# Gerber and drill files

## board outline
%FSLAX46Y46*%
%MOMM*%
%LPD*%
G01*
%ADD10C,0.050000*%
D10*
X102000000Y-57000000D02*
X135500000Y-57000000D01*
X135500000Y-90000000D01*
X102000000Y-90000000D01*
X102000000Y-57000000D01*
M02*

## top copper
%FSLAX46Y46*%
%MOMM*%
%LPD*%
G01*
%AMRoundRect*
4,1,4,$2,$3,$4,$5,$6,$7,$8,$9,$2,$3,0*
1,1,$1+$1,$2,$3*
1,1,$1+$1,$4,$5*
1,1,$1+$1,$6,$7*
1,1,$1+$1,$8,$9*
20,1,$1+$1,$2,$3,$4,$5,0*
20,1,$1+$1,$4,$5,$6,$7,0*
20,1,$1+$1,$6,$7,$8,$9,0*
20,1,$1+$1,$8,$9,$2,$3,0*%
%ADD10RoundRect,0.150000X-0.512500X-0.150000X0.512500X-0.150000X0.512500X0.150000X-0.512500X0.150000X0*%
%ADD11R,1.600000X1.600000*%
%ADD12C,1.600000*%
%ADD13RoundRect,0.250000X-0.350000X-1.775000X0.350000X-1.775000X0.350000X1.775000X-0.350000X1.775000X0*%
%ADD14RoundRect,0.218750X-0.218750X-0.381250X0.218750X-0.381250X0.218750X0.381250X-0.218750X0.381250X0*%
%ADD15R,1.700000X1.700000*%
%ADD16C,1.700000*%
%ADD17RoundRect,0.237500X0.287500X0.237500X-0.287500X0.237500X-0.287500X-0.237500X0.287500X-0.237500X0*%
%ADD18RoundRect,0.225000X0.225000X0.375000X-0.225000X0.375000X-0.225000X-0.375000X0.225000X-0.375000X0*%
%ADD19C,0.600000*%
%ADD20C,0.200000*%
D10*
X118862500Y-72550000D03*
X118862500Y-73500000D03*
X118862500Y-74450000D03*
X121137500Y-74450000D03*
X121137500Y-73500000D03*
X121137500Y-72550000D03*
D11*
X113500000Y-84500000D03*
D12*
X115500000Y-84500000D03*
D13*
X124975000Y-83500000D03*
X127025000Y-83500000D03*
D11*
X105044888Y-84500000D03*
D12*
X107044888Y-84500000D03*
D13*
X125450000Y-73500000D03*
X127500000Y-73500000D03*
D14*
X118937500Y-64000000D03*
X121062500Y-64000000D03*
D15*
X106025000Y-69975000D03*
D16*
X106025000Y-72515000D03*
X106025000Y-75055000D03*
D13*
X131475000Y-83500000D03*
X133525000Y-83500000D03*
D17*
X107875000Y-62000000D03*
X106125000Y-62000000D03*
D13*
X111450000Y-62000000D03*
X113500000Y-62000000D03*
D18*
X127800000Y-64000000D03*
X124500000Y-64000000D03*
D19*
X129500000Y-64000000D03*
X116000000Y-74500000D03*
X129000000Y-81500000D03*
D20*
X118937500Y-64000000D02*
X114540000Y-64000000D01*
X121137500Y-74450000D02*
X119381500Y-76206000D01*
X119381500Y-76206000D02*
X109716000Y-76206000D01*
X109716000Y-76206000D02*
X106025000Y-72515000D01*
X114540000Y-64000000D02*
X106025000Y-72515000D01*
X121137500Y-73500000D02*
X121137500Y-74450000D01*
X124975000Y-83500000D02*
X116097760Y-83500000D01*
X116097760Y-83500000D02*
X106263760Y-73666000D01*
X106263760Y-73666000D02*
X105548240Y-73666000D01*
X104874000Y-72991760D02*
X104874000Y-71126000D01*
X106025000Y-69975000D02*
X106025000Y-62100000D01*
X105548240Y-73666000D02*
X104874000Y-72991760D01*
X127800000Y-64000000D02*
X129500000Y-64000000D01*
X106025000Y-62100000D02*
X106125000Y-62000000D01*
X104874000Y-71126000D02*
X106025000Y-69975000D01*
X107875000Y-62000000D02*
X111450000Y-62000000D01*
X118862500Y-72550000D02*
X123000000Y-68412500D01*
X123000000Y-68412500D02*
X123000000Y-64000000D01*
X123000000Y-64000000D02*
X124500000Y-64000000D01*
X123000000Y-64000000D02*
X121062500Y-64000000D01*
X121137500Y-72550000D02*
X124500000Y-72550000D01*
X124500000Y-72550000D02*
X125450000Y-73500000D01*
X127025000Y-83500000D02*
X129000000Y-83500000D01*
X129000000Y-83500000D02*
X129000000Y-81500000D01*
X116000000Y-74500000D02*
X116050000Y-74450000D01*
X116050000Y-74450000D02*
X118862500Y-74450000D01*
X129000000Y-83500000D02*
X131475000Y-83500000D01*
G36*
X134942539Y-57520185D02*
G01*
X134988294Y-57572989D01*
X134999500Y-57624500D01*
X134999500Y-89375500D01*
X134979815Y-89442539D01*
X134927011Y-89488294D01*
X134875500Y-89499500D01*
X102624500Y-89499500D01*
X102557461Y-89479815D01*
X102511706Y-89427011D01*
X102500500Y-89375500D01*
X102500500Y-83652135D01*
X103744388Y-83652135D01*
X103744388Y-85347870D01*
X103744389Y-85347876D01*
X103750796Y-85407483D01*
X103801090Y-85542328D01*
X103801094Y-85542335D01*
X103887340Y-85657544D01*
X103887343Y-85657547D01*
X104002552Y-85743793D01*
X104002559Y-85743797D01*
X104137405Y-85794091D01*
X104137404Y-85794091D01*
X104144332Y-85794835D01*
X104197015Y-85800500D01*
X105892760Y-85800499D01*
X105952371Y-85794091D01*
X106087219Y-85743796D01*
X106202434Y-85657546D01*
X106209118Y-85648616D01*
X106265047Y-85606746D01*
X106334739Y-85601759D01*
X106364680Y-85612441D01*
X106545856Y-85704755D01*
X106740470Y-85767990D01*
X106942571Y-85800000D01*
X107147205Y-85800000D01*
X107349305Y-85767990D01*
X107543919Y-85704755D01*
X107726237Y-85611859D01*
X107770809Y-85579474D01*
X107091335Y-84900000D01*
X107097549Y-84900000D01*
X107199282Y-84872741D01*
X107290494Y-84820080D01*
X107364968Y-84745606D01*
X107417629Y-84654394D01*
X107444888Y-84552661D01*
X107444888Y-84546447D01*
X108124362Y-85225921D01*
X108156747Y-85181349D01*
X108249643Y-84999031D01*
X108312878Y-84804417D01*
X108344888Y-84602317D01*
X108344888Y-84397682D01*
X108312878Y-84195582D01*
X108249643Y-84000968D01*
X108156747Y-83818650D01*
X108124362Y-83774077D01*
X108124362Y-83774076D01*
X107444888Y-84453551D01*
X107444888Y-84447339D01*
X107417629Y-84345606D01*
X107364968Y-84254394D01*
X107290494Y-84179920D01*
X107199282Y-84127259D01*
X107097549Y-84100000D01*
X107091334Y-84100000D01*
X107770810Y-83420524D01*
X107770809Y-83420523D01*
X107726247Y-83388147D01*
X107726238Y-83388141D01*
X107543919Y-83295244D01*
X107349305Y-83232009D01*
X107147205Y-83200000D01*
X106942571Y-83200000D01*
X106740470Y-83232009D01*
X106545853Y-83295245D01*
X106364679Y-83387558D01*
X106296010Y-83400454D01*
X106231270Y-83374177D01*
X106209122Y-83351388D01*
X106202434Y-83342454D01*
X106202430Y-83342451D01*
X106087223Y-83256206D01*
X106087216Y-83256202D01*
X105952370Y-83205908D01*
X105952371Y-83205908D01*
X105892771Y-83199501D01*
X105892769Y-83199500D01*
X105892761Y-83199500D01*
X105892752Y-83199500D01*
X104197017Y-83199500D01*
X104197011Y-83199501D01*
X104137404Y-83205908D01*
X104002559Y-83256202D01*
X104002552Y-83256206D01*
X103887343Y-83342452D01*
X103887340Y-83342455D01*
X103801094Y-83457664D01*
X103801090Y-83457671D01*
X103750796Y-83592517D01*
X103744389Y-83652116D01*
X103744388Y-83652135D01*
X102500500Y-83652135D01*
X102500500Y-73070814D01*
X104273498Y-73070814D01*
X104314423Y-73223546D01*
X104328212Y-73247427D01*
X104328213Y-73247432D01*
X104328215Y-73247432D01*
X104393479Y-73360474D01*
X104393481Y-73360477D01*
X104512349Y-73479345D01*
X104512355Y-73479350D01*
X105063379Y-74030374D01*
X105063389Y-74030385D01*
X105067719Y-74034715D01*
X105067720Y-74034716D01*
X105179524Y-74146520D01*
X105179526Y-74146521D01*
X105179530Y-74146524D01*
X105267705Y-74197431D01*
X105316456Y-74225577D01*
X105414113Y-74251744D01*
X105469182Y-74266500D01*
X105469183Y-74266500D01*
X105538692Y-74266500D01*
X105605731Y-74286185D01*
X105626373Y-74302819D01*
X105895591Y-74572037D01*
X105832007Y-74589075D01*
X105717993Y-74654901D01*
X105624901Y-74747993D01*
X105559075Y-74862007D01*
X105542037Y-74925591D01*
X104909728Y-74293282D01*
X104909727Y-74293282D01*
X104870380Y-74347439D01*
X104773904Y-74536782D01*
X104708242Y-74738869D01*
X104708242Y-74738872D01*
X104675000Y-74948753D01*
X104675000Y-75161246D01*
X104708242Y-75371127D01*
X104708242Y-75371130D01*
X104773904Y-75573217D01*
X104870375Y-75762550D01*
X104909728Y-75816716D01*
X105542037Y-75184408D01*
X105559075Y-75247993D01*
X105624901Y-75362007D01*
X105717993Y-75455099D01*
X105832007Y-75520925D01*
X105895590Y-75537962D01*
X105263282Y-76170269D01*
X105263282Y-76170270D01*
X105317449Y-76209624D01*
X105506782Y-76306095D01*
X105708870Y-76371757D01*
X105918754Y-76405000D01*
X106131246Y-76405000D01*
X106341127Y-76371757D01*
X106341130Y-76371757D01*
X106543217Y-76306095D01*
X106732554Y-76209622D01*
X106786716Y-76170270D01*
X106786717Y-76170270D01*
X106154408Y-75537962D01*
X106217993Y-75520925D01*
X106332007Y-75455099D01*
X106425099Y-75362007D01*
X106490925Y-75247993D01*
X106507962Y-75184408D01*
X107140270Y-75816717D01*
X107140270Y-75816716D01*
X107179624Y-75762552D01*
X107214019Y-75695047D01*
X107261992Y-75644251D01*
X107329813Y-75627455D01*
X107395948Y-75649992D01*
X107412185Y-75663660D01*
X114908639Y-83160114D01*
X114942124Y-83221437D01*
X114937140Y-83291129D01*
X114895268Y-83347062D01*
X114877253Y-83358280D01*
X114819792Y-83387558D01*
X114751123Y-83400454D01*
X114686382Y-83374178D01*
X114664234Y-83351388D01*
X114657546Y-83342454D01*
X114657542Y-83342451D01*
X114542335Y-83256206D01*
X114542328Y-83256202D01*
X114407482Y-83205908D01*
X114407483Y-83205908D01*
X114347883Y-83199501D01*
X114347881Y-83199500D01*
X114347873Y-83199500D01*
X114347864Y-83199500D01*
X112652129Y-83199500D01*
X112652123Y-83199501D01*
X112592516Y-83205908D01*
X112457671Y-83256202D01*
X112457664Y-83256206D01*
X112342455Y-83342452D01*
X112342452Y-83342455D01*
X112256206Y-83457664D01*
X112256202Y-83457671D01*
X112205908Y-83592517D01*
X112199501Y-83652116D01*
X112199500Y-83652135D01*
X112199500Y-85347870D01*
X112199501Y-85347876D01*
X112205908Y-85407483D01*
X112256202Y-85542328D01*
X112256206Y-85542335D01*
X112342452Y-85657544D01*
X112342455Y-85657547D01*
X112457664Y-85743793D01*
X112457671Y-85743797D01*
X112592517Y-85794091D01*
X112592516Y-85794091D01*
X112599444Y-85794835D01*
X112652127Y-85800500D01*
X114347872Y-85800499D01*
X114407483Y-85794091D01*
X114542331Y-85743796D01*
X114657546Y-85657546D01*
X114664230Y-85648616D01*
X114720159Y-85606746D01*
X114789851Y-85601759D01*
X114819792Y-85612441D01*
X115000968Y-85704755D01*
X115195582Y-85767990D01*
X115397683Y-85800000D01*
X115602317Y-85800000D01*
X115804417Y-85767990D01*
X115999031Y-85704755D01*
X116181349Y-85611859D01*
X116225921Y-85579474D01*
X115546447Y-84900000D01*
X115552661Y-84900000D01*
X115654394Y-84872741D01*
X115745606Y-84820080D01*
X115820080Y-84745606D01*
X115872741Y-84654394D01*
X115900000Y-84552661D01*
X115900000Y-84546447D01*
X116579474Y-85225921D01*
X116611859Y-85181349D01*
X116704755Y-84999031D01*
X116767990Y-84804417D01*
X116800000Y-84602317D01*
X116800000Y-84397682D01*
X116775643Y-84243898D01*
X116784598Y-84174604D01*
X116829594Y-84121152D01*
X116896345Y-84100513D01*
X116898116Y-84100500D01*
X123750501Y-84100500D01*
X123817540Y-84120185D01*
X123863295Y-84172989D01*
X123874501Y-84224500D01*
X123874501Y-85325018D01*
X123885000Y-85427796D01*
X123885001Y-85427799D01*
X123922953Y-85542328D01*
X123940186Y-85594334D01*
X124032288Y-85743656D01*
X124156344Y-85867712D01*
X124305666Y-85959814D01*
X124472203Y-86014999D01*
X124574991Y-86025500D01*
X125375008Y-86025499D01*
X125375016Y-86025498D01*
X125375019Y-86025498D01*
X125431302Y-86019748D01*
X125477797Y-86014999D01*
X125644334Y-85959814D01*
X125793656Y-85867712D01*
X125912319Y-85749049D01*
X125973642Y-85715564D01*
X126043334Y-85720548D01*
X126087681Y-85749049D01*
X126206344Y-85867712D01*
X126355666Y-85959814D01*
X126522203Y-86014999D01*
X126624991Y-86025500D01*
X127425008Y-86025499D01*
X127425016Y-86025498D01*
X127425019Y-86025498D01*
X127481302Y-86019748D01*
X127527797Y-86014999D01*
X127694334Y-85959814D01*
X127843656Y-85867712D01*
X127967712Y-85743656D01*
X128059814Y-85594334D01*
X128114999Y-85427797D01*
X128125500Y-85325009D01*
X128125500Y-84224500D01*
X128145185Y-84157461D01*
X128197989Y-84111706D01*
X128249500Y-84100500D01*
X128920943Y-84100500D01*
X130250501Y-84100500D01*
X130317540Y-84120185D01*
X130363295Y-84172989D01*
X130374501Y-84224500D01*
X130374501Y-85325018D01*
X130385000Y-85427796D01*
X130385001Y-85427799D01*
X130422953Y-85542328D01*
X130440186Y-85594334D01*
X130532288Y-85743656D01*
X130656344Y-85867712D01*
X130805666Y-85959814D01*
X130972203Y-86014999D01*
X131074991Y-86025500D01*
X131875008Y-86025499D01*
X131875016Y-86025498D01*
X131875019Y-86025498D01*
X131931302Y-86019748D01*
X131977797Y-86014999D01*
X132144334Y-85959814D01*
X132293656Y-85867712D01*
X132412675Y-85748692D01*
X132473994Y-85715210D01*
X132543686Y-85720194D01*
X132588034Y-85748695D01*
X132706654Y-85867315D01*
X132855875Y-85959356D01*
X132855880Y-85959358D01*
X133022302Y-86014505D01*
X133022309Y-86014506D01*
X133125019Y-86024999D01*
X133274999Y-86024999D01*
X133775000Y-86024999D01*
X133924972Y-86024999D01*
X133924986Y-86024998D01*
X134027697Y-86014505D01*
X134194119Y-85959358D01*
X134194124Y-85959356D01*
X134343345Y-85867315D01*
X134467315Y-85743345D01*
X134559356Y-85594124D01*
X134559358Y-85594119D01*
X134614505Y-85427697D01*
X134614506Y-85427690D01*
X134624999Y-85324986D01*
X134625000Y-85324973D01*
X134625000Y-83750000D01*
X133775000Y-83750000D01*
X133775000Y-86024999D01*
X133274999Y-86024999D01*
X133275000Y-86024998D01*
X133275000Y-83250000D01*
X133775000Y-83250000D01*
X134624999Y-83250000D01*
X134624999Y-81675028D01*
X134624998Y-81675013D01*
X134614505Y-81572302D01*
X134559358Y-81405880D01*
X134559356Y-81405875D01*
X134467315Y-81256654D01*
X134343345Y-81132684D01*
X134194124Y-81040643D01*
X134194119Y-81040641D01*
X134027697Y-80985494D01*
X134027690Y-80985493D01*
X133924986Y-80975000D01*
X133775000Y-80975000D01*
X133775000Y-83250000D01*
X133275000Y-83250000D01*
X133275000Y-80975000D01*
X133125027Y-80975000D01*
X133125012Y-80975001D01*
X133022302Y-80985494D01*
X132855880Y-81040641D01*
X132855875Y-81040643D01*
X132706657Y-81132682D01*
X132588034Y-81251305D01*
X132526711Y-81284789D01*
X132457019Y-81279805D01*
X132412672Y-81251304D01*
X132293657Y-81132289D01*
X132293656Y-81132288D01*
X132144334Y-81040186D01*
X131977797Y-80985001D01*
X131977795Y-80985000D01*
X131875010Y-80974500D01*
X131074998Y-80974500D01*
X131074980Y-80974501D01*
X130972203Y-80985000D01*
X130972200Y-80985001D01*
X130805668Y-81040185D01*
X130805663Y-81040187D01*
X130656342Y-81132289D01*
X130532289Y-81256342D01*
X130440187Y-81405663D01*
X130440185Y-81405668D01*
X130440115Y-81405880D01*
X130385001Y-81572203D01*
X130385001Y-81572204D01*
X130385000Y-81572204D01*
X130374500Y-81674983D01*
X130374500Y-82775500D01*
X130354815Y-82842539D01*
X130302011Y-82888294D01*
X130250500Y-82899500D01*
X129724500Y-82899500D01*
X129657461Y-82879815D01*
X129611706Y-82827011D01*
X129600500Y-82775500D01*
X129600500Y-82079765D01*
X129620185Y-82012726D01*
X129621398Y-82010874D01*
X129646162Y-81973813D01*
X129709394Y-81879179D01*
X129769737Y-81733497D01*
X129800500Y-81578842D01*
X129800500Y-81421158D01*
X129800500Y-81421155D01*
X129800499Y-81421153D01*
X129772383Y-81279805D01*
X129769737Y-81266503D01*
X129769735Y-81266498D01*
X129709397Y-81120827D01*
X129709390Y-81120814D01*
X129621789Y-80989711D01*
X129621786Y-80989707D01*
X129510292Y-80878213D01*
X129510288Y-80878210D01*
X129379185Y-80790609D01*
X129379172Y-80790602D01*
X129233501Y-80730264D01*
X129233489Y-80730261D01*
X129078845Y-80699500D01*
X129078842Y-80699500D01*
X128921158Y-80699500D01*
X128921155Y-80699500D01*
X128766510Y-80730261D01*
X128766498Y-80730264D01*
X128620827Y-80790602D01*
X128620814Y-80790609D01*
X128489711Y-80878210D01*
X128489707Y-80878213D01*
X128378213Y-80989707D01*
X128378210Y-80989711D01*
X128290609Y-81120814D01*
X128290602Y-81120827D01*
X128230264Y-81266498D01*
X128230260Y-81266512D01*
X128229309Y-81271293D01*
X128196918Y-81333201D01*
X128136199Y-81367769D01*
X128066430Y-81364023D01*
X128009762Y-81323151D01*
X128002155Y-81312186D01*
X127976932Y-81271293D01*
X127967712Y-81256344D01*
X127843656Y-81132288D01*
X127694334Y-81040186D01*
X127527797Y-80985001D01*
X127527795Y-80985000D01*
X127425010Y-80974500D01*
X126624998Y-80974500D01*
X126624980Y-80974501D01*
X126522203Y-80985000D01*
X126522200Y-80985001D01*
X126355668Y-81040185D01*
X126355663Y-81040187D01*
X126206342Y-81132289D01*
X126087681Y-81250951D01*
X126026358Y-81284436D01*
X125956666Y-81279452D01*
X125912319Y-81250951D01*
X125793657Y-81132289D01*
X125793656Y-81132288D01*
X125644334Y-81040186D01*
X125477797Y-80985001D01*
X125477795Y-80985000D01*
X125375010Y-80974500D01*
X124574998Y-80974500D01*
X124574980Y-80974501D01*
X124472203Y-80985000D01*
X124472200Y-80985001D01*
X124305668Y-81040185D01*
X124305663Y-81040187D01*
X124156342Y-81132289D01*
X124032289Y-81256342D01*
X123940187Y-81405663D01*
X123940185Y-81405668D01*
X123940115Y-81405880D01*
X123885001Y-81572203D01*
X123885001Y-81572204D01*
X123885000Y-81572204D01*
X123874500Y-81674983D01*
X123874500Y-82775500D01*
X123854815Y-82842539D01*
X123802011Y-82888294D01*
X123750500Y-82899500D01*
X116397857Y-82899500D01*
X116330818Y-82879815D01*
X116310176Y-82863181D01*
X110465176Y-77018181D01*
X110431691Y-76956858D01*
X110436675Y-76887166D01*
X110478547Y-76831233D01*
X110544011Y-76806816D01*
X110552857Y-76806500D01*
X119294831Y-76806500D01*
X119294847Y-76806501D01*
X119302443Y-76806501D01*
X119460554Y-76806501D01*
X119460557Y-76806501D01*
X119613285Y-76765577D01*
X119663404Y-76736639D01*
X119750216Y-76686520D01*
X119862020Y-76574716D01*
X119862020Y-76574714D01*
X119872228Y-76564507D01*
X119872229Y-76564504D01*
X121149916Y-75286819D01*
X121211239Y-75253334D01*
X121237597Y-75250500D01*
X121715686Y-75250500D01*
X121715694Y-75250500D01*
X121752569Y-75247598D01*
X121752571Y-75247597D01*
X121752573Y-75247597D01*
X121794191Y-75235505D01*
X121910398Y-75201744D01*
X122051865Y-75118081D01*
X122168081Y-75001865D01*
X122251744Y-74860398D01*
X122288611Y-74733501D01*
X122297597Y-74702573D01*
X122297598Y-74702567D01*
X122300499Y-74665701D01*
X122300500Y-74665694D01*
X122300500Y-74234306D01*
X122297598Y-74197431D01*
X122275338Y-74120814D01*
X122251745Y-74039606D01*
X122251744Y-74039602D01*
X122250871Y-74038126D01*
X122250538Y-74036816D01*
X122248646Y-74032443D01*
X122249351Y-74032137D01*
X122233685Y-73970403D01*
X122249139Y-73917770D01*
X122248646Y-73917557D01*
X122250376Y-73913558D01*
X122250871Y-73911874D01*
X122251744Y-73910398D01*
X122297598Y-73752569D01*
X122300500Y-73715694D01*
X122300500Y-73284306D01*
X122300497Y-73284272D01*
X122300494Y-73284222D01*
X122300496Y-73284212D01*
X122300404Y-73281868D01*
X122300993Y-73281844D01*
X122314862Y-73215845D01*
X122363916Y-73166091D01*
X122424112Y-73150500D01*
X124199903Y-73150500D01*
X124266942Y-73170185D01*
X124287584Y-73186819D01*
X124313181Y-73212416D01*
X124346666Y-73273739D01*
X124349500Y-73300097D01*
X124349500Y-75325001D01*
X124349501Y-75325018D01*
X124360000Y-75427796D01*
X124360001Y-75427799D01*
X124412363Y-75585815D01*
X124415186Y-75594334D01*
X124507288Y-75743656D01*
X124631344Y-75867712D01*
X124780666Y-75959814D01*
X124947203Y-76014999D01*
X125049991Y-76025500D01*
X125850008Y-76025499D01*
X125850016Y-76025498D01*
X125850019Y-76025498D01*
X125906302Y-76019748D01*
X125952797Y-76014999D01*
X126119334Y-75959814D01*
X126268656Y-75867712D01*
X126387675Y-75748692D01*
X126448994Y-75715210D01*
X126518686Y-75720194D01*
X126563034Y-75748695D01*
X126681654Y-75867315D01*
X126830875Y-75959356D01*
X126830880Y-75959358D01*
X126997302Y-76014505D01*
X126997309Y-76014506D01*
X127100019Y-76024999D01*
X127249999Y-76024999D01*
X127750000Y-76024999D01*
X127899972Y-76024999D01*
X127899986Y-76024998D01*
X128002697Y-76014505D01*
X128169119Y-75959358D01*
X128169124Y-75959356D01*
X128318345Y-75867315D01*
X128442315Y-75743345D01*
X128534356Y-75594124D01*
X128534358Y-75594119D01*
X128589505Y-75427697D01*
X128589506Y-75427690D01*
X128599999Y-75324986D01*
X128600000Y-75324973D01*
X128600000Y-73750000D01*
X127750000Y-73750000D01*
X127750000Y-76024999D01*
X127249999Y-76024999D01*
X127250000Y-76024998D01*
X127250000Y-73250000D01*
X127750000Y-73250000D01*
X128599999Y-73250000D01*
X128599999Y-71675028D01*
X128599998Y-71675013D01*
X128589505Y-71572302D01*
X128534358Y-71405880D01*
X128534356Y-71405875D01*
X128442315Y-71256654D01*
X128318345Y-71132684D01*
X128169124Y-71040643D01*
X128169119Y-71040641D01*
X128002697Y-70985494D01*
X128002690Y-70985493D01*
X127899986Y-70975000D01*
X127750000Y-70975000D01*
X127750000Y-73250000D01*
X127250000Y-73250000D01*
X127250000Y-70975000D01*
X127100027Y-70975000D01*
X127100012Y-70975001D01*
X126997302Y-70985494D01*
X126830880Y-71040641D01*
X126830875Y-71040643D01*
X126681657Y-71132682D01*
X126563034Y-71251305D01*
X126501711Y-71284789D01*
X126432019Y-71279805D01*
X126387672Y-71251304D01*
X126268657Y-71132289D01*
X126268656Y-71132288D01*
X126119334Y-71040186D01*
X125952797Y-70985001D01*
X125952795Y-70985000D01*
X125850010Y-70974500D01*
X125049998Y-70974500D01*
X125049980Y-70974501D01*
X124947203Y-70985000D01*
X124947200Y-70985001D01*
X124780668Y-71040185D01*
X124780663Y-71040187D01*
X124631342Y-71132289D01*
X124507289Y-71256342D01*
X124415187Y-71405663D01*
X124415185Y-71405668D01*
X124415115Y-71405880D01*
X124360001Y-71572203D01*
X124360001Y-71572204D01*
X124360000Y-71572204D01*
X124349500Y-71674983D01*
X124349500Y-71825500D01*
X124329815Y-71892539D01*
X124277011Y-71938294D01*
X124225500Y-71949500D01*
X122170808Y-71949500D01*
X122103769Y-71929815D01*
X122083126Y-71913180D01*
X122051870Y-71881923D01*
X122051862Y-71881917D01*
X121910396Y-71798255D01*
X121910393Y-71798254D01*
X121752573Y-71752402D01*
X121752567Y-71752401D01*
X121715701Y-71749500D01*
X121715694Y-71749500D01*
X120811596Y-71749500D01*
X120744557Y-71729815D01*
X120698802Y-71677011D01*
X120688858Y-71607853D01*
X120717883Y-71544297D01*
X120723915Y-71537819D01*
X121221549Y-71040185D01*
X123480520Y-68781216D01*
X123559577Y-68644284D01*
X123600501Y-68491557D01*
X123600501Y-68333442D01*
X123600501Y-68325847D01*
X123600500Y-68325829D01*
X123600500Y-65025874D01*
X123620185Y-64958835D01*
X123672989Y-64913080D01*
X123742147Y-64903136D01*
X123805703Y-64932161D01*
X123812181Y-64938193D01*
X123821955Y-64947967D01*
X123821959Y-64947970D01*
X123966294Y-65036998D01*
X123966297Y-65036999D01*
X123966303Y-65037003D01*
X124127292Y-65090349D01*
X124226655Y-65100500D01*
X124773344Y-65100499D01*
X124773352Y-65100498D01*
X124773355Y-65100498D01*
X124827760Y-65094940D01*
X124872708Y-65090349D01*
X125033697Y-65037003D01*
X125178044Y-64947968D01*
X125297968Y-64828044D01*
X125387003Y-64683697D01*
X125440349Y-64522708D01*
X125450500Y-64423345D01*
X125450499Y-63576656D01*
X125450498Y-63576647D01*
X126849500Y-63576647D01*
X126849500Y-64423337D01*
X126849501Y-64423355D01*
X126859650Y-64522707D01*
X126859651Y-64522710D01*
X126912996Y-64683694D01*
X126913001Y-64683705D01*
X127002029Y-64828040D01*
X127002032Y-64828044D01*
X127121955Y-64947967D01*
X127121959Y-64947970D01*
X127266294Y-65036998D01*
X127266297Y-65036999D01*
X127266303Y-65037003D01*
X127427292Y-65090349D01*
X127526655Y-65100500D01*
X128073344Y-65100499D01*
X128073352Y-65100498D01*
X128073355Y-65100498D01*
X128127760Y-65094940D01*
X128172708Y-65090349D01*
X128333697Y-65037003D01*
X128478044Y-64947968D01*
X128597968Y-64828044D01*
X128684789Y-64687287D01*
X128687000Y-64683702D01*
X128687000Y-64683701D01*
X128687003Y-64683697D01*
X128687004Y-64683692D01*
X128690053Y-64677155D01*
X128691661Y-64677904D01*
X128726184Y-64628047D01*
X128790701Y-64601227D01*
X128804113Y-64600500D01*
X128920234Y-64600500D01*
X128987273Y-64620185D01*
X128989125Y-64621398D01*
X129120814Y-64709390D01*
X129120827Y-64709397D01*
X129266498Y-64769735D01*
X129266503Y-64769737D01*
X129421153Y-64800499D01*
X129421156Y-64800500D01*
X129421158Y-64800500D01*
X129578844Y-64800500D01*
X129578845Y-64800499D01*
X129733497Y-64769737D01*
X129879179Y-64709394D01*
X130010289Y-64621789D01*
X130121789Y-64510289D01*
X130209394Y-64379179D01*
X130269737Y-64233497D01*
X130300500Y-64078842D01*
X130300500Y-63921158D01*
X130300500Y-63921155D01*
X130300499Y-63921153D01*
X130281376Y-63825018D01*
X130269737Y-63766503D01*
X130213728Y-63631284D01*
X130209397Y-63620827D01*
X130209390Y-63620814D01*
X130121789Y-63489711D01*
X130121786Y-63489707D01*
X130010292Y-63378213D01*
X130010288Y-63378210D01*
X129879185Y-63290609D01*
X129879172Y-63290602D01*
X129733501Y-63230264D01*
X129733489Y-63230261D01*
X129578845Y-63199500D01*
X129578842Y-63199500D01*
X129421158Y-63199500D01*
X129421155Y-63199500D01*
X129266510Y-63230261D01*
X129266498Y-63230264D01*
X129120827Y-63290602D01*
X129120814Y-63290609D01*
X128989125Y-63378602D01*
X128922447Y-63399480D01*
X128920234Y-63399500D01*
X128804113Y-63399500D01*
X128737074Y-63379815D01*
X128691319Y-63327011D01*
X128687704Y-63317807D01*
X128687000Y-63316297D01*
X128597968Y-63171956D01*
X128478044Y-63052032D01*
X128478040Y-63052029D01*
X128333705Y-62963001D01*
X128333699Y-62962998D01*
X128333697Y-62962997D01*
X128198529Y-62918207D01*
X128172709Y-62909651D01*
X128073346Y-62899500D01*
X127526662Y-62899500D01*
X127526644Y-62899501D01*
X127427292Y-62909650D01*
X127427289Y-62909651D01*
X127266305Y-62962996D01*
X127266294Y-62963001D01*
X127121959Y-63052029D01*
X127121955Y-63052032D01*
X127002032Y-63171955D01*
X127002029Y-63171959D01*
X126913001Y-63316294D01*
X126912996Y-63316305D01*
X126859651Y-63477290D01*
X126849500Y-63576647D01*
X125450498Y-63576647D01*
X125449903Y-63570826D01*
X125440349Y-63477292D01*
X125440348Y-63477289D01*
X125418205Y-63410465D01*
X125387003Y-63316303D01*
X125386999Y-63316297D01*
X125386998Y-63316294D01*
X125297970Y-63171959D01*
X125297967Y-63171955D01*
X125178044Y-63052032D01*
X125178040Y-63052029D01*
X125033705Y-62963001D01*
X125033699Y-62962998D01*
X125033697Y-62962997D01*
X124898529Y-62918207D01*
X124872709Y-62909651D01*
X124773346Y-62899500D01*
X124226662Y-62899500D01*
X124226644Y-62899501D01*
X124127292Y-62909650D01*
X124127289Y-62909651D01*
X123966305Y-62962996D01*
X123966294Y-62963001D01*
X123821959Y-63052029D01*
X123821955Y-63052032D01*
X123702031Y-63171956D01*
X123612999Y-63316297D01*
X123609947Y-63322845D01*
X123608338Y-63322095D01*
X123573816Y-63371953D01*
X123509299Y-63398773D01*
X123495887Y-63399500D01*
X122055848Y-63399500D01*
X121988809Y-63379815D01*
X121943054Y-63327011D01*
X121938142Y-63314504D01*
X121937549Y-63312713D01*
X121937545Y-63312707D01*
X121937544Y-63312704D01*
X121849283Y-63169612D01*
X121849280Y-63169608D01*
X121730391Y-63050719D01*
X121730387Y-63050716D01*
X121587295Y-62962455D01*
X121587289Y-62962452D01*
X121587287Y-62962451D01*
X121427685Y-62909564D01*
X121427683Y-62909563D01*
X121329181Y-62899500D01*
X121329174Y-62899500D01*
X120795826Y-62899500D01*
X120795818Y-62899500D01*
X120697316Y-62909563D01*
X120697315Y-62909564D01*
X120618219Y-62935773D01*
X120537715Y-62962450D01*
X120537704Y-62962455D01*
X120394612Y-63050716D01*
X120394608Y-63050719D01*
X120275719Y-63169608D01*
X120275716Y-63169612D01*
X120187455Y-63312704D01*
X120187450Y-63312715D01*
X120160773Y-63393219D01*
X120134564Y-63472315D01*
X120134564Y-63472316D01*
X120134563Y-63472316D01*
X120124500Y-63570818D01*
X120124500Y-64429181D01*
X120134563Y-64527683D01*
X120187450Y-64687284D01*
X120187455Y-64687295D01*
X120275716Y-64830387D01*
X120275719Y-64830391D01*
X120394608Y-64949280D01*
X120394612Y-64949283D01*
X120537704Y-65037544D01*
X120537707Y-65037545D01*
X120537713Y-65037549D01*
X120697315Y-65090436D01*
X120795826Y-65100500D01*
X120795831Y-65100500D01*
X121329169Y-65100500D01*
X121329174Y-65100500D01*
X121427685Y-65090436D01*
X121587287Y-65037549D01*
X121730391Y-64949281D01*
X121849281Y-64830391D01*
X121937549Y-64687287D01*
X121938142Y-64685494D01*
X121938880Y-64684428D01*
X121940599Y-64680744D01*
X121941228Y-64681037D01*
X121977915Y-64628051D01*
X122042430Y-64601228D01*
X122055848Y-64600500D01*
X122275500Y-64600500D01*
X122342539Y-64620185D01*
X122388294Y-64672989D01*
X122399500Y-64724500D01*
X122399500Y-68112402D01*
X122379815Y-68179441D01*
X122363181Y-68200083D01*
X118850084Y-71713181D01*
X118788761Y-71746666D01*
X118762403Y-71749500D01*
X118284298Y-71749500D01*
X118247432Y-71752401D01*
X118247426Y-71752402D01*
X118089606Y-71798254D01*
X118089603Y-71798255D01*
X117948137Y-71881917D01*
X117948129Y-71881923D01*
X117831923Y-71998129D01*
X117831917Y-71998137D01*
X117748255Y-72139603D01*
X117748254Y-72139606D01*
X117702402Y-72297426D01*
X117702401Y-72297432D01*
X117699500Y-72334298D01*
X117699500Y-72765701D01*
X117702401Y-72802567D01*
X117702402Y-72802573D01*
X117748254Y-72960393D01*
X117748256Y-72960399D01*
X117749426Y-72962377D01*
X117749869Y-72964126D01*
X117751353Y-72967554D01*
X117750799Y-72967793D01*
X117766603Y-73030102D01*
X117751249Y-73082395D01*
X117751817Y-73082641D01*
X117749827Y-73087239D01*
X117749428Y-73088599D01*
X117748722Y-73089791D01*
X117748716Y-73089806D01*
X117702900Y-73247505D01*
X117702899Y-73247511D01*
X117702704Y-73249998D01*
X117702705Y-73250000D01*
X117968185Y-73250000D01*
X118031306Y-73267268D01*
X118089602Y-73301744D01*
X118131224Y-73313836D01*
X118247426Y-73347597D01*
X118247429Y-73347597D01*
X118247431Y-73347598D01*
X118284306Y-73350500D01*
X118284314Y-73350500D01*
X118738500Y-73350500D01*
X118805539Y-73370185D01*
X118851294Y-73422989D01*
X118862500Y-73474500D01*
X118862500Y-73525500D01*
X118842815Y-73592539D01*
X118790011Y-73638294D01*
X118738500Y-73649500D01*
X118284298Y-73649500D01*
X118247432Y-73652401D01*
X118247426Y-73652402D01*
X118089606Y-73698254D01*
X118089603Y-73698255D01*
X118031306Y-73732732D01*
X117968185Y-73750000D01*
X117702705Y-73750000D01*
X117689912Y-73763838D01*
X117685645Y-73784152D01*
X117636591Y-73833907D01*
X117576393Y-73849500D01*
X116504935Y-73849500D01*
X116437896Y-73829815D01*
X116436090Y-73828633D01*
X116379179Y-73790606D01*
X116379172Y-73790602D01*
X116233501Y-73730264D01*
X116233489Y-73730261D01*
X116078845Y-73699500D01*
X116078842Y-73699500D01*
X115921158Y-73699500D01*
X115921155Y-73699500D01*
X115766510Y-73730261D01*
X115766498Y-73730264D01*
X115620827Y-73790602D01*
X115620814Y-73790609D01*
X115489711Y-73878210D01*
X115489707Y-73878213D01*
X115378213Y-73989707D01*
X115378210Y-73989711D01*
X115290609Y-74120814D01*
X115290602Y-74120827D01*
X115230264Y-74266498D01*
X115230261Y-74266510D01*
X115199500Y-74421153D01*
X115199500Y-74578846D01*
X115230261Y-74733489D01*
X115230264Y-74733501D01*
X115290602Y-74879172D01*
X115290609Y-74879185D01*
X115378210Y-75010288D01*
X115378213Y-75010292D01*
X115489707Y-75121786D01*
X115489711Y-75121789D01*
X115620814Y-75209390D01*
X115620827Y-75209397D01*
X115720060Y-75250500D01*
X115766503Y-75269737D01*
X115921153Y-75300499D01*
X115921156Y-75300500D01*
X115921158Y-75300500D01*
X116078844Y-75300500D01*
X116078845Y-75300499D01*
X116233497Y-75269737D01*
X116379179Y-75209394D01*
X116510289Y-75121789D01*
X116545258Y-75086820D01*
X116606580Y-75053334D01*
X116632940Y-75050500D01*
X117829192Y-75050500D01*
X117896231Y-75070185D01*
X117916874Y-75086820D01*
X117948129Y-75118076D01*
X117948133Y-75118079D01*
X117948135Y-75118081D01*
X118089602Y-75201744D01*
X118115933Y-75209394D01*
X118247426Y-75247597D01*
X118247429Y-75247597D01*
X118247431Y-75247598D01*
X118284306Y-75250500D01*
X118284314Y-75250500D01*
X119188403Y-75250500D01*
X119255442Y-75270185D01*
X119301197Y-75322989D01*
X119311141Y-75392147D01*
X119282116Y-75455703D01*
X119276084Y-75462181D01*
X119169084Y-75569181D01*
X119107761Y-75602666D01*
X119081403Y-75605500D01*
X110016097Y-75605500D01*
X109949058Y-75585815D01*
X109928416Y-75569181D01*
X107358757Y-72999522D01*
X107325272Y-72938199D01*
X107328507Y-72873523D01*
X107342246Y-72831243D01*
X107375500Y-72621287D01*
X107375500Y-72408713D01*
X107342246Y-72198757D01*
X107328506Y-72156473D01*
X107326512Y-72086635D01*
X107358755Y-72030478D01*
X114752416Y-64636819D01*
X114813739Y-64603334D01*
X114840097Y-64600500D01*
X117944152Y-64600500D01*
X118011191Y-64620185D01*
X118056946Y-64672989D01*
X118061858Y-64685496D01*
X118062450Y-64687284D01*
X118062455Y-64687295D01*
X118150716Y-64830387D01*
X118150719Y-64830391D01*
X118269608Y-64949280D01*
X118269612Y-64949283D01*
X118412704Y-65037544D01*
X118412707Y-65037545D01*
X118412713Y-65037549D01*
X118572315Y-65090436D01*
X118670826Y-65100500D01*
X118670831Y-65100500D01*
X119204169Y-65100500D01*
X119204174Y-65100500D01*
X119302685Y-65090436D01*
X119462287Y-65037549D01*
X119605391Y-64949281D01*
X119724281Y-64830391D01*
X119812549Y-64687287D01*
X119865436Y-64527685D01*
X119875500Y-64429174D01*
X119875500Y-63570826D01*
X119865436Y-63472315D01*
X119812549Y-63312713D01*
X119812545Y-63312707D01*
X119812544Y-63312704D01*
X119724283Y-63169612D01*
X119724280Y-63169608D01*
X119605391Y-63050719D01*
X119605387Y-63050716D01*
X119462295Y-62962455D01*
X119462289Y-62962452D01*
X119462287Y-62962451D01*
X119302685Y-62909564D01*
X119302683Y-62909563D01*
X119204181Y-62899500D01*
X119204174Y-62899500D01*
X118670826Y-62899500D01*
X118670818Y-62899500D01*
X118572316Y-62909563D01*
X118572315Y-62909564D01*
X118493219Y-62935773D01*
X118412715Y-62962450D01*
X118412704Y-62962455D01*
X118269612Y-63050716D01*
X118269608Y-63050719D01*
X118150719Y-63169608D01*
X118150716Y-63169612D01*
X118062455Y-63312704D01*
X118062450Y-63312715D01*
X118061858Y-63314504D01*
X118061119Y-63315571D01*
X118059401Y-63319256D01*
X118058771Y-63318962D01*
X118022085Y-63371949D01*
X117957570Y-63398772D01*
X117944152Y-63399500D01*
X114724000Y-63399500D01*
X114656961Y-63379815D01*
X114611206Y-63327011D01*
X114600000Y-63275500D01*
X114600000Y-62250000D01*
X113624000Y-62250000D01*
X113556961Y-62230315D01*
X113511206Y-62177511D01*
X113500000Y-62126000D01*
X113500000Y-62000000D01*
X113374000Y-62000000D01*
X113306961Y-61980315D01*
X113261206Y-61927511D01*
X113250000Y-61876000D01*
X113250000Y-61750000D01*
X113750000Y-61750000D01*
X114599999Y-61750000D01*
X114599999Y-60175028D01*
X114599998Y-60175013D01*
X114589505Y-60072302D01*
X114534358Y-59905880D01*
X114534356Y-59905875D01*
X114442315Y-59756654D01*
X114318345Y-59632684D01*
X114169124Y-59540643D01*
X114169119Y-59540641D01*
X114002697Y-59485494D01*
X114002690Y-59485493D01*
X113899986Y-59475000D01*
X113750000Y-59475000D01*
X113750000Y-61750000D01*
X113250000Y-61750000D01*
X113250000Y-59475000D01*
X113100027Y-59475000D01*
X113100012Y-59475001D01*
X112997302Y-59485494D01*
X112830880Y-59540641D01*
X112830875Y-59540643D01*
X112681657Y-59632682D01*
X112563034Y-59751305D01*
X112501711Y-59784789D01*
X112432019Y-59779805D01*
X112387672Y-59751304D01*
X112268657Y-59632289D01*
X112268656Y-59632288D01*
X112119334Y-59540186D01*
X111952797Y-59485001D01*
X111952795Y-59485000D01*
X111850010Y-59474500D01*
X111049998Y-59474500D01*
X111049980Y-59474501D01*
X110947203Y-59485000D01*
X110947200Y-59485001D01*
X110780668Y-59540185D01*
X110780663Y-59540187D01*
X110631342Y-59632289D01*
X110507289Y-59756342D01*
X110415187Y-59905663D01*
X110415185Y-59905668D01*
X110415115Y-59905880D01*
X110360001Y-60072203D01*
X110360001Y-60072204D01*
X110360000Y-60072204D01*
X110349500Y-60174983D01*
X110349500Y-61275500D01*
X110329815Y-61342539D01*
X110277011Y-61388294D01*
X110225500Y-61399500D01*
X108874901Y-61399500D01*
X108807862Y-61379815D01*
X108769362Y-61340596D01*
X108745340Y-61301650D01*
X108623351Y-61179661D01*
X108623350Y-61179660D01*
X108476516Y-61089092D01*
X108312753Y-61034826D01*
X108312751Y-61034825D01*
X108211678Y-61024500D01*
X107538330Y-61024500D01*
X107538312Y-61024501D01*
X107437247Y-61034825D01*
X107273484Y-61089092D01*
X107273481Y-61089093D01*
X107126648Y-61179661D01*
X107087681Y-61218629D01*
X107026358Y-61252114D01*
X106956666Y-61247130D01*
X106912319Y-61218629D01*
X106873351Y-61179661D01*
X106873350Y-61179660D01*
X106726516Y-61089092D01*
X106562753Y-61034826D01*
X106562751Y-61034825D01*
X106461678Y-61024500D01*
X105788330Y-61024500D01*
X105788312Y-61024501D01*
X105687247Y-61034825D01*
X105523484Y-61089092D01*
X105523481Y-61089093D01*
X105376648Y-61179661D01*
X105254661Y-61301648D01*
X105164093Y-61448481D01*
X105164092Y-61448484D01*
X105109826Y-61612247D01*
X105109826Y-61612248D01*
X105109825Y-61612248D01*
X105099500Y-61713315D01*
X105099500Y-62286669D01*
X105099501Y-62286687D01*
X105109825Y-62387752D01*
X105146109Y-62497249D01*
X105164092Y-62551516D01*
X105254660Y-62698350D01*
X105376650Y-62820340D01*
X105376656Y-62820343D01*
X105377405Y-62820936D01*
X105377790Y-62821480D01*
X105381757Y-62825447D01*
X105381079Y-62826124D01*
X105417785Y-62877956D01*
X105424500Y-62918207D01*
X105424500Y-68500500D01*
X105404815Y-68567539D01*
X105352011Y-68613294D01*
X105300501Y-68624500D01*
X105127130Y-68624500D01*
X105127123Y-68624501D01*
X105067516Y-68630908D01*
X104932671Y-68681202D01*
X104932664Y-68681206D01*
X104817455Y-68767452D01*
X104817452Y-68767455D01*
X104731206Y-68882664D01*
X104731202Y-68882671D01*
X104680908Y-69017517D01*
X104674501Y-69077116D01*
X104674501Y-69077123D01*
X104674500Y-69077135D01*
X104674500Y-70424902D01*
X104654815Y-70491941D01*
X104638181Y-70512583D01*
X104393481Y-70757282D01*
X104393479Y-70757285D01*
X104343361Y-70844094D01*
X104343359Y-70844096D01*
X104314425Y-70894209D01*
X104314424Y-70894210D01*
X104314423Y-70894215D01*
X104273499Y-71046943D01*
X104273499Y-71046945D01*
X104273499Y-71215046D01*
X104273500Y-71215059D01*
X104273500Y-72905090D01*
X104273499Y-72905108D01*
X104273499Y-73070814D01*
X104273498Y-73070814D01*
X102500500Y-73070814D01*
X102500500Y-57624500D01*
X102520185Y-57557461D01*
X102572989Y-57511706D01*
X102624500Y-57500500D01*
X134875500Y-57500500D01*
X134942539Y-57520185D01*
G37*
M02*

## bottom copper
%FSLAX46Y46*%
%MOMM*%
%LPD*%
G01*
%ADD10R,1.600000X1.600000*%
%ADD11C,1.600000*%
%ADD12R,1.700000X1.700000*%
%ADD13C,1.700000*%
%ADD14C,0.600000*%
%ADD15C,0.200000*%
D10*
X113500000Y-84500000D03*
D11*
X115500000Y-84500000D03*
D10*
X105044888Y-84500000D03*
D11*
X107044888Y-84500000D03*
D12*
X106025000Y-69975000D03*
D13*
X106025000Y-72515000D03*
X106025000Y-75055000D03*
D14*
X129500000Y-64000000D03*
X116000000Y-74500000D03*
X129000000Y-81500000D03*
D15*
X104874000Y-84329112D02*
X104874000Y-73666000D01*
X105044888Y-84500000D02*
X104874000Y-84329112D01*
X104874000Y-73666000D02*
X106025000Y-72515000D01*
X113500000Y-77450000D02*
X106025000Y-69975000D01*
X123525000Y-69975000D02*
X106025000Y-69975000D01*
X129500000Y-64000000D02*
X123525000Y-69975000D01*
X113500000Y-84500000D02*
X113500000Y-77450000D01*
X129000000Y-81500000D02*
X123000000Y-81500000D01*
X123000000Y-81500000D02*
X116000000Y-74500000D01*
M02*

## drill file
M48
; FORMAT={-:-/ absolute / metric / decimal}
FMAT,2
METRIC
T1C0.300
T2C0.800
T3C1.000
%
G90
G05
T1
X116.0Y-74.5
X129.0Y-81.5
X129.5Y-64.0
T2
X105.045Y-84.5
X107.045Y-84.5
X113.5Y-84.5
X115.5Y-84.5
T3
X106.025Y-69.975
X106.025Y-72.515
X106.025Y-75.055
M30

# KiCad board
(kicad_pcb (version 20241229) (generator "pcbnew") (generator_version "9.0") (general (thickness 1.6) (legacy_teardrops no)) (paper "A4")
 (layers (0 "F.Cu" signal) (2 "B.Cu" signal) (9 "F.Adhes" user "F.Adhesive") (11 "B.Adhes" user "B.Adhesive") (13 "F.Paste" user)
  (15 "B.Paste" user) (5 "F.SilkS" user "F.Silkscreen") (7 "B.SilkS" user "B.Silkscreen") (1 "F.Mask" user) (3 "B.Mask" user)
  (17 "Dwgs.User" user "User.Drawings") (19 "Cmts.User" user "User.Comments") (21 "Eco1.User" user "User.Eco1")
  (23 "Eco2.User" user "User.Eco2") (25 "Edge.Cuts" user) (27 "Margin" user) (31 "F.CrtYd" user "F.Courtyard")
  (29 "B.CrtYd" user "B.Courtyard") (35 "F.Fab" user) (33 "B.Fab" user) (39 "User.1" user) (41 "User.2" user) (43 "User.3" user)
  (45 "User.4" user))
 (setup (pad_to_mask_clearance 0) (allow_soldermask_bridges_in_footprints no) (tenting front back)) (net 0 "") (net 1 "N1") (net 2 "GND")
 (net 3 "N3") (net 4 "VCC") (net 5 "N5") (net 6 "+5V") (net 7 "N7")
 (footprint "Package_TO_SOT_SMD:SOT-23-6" (layer "F.Cu") (at 120 73.5)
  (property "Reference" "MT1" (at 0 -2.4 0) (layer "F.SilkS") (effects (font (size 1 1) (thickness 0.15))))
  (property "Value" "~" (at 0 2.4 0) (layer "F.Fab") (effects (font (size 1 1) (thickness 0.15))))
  (pad "1" smd roundrect (at -1.1375 -0.95) (size 1.325 0.6) (layers "F.Cu" "F.Mask" "F.Paste") (roundrect_rratio 0.25) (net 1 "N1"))
  (pad "2" smd roundrect (at -1.1375 0) (size 1.325 0.6) (layers "F.Cu" "F.Mask" "F.Paste") (roundrect_rratio 0.25) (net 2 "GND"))
  (pad "3" smd roundrect (at -1.1375 0.95) (size 1.325 0.6) (layers "F.Cu" "F.Mask" "F.Paste") (roundrect_rratio 0.25) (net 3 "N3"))
  (pad "4" smd roundrect (at 1.1375 0.95) (size 1.325 0.6) (layers "F.Cu" "F.Mask" "F.Paste") (roundrect_rratio 0.25) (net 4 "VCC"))
  (pad "5" smd roundrect (at 1.1375 0) (size 1.325 0.6) (layers "F.Cu" "F.Mask" "F.Paste") (roundrect_rratio 0.25) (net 4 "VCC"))
  (pad "6" smd roundrect (at 1.1375 -0.95) (size 1.325 0.6) (layers "F.Cu" "F.Mask" "F.Paste") (roundrect_rratio 0.25) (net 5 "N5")))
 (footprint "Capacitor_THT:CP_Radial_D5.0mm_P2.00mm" (layer "F.Cu") (at 113.5 84.5)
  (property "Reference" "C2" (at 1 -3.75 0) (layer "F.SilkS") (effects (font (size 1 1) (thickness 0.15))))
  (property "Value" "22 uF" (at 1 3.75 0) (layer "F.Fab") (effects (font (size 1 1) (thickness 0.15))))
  (pad "1" thru_hole rect (at 0 0) (size 1.6 1.6) (drill 0.8) (layers "*.Cu" "*.Mask") (remove_unused_layers no) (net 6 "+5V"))
  (pad "2" thru_hole circle (at 2 0) (size 1.6 1.6) (drill 0.8) (layers "*.Cu" "*.Mask") (remove_unused_layers no) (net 2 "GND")))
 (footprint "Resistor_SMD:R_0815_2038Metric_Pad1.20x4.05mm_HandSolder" (layer "F.Cu") (at 126 83.5)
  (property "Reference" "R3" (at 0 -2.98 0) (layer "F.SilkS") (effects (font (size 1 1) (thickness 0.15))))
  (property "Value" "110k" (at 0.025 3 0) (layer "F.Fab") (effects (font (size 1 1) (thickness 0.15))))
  (pad "1" smd roundrect (at -1.025 0) (size 1.2 4.05) (layers "F.Cu" "F.Mask" "F.Paste") (roundrect_rratio 0.208333) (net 6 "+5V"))
  (pad "2" smd roundrect (at 1.025 0) (size 1.2 4.05) (layers "F.Cu" "F.Mask" "F.Paste") (roundrect_rratio 0.208333) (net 3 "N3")))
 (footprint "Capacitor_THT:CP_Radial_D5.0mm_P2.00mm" (layer "F.Cu") (at 105.044888 84.5)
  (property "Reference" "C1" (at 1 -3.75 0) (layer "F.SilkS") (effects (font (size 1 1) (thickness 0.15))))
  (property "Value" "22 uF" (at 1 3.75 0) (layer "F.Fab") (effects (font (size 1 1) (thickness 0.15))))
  (pad "1" thru_hole rect (at 0 0) (size 1.6 1.6) (drill 0.8) (layers "*.Cu" "*.Mask") (remove_unused_layers no) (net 4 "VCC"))
  (pad "2" thru_hole circle (at 2 0) (size 1.6 1.6) (drill 0.8) (layers "*.Cu" "*.Mask") (remove_unused_layers no) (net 2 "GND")))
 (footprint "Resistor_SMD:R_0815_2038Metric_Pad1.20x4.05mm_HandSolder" (layer "F.Cu") (at 126.475 73.5)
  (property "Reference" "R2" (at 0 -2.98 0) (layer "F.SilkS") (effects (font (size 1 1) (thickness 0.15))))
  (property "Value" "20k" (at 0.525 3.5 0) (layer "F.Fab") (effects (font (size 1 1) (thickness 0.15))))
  (pad "1" smd roundrect (at -1.025 0) (size 1.2 4.05) (layers "F.Cu" "F.Mask" "F.Paste") (roundrect_rratio 0.208333) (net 5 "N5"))
  (pad "2" smd roundrect (at 1.025 0) (size 1.2 4.05) (layers "F.Cu" "F.Mask" "F.Paste") (roundrect_rratio 0.208333) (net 2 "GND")))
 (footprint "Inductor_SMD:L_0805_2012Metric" (layer "F.Cu") (at 120 64)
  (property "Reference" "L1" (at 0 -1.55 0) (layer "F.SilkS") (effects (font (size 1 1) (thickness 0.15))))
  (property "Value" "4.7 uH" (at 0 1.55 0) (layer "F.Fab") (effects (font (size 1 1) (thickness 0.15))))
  (pad "1" smd roundrect (at -1.0625 0) (size 0.875 1.2) (layers "F.Cu" "F.Mask" "F.Paste") (roundrect_rratio 0.25) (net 4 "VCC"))
  (pad "2" smd roundrect (at 1.0625 0) (size 0.875 1.2) (layers "F.Cu" "F.Mask" "F.Paste") (roundrect_rratio 0.25) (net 1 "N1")))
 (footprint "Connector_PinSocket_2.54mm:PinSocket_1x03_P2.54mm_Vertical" (layer "F.Cu") (at 106.025 69.975)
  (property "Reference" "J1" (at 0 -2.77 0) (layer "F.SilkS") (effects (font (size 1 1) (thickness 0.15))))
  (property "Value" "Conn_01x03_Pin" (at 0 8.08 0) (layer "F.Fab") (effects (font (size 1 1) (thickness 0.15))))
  (pad "1" thru_hole rect (at 0 0) (size 1.7 1.7) (drill 1) (layers "*.Cu" "*.Mask") (remove_unused_layers no) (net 6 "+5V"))
  (pad "2" thru_hole circle (at 0 2.54) (size 1.7 1.7) (drill 1) (layers "*.Cu" "*.Mask") (remove_unused_layers no) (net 4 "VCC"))
  (pad "3" thru_hole circle (at 0 5.08) (size 1.7 1.7) (drill 1) (layers "*.Cu" "*.Mask") (remove_unused_layers no) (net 2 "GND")))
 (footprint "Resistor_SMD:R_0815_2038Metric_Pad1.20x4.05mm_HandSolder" (layer "F.Cu") (at 132.5 83.5)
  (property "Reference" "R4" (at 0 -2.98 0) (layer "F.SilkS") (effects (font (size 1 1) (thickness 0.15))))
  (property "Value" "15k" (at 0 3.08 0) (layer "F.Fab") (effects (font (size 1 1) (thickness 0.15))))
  (pad "1" smd roundrect (at -1.025 0) (size 1.2 4.05) (layers "F.Cu" "F.Mask" "F.Paste") (roundrect_rratio 0.208333) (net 3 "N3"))
  (pad "2" smd roundrect (at 1.025 0) (size 1.2 4.05) (layers "F.Cu" "F.Mask" "F.Paste") (roundrect_rratio 0.208333) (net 2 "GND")))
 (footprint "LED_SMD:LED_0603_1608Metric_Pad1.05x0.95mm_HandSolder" (layer "F.Cu") (at 107 62 180)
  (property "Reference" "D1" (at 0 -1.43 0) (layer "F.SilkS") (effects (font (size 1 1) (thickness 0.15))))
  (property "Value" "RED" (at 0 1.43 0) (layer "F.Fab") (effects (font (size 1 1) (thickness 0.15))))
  (pad "1" smd roundrect (at -0.875 0 180) (size 1.05 0.95) (layers "F.Cu" "F.Mask" "F.Paste") (roundrect_rratio 0.25) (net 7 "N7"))
  (pad "2" smd roundrect (at 0.875 0 180) (size 1.05 0.95) (layers "F.Cu" "F.Mask" "F.Paste") (roundrect_rratio 0.25) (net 6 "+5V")))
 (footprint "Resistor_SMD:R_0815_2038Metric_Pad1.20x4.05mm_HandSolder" (layer "F.Cu") (at 112.475 62)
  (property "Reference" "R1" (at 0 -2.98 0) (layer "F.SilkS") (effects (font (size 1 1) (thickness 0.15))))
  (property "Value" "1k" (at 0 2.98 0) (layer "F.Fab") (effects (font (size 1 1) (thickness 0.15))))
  (pad "1" smd roundrect (at -1.025 0) (size 1.2 4.05) (layers "F.Cu" "F.Mask" "F.Paste") (roundrect_rratio 0.208333) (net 7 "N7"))
  (pad "2" smd roundrect (at 1.025 0) (size 1.2 4.05) (layers "F.Cu" "F.Mask" "F.Paste") (roundrect_rratio 0.208333) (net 2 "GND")))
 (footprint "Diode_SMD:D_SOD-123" (layer "F.Cu") (at 126.15 64 180)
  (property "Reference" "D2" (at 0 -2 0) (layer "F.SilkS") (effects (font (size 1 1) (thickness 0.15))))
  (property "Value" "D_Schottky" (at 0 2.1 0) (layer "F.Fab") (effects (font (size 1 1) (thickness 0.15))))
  (pad "1" smd roundrect (at -1.65 0 180) (size 0.9 1.2) (layers "F.Cu" "F.Mask" "F.Paste") (roundrect_rratio 0.25) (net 6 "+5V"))
  (pad "2" smd roundrect (at 1.65 0 180) (size 0.9 1.2) (layers "F.Cu" "F.Mask" "F.Paste") (roundrect_rratio 0.25) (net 1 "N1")))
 (gr_rect (start 102 57) (end 135.5 90) (stroke (width 0.05) (type default)) (fill no) (layer "Edge.Cuts"))
 (segment (start 118.9375 64) (end 114.54 64) (width 0.2) (layer "F.Cu") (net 4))
 (segment (start 121.1375 74.45) (end 119.3815 76.206) (width 0.2) (layer "F.Cu") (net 4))
 (segment (start 119.3815 76.206) (end 109.716 76.206) (width 0.2) (layer "F.Cu") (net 4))
 (segment (start 109.716 76.206) (end 106.025 72.515) (width 0.2) (layer "F.Cu") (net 4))
 (segment (start 114.54 64) (end 106.025 72.515) (width 0.2) (layer "F.Cu") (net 4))
 (segment (start 121.1375 73.5) (end 121.1375 74.45) (width 0.2) (layer "F.Cu") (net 4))
 (segment (start 104.874 84.329112) (end 104.874 73.666) (width 0.2) (layer "B.Cu") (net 4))
 (segment (start 105.044888 84.5) (end 104.874 84.329112) (width 0.2) (layer "B.Cu") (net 4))
 (segment (start 104.874 73.666) (end 106.025 72.515) (width 0.2) (layer "B.Cu") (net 4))
 (segment (start 124.975 83.5) (end 116.09776 83.5) (width 0.2) (layer "F.Cu") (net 6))
 (segment (start 116.09776 83.5) (end 106.26376 73.666) (width 0.2) (layer "F.Cu") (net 6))
 (segment (start 106.26376 73.666) (end 105.54824 73.666) (width 0.2) (layer "F.Cu") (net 6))
 (segment (start 104.874 72.99176) (end 104.874 71.126) (width 0.2) (layer "F.Cu") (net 6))
 (segment (start 106.025 69.975) (end 106.025 62.1) (width 0.2) (layer "F.Cu") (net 6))
 (segment (start 105.54824 73.666) (end 104.874 72.99176) (width 0.2) (layer "F.Cu") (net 6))
 (segment (start 127.8 64) (end 129.5 64) (width 0.2) (layer "F.Cu") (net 6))
 (segment (start 106.025 62.1) (end 106.125 62) (width 0.2) (layer "F.Cu") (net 6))
 (segment (start 104.874 71.126) (end 106.025 69.975) (width 0.2) (layer "F.Cu") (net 6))
 (via (at 129.5 64) (size 0.6) (drill 0.3) (layers "F.Cu" "B.Cu") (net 6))
 (segment (start 113.5 77.45) (end 106.025 69.975) (width 0.2) (layer "B.Cu") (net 6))
 (segment (start 123.525 69.975) (end 106.025 69.975) (width 0.2) (layer "B.Cu") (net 6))
 (segment (start 129.5 64) (end 123.525 69.975) (width 0.2) (layer "B.Cu") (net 6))
 (segment (start 113.5 84.5) (end 113.5 77.45) (width 0.2) (layer "B.Cu") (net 6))
 (segment (start 107.875 62) (end 111.45 62) (width 0.2) (layer "F.Cu") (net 7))
 (segment (start 118.8625 72.55) (end 123 68.4125) (width 0.2) (layer "F.Cu") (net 1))
 (segment (start 123 68.4125) (end 123 64) (width 0.2) (layer "F.Cu") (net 1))
 (segment (start 123 64) (end 124.5 64) (width 0.2) (layer "F.Cu") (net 1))
 (segment (start 123 64) (end 121.0625 64) (width 0.2) (layer "F.Cu") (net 1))
 (segment (start 121.1375 72.55) (end 124.5 72.55) (width 0.2) (layer "F.Cu") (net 5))
 (segment (start 124.5 72.55) (end 125.45 73.5) (width 0.2) (layer "F.Cu") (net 5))
 (segment (start 127.025 83.5) (end 129 83.5) (width 0.2) (layer "F.Cu") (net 3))
 (segment (start 129 83.5) (end 129 81.5) (width 0.2) (layer "F.Cu") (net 3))
 (segment (start 116 74.5) (end 116.05 74.45) (width 0.2) (layer "F.Cu") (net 3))
 (segment (start 116.05 74.45) (end 118.8625 74.45) (width 0.2) (layer "F.Cu") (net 3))
 (segment (start 129 83.5) (end 131.475 83.5) (width 0.2) (layer "F.Cu") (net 3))
 (via (at 116 74.5) (size 0.6) (drill 0.3) (layers "F.Cu" "B.Cu") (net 3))
 (via (at 129 81.5) (size 0.6) (drill 0.3) (layers "F.Cu" "B.Cu") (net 3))
 (segment (start 129 81.5) (end 123 81.5) (width 0.2) (layer "B.Cu") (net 3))
 (segment (start 123 81.5) (end 116 74.5) (width 0.2) (layer "B.Cu") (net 3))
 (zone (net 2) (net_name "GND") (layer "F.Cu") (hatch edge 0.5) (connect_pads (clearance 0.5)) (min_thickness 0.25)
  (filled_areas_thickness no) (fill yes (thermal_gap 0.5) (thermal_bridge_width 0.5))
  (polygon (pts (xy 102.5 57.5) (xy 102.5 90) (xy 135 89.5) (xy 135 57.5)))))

